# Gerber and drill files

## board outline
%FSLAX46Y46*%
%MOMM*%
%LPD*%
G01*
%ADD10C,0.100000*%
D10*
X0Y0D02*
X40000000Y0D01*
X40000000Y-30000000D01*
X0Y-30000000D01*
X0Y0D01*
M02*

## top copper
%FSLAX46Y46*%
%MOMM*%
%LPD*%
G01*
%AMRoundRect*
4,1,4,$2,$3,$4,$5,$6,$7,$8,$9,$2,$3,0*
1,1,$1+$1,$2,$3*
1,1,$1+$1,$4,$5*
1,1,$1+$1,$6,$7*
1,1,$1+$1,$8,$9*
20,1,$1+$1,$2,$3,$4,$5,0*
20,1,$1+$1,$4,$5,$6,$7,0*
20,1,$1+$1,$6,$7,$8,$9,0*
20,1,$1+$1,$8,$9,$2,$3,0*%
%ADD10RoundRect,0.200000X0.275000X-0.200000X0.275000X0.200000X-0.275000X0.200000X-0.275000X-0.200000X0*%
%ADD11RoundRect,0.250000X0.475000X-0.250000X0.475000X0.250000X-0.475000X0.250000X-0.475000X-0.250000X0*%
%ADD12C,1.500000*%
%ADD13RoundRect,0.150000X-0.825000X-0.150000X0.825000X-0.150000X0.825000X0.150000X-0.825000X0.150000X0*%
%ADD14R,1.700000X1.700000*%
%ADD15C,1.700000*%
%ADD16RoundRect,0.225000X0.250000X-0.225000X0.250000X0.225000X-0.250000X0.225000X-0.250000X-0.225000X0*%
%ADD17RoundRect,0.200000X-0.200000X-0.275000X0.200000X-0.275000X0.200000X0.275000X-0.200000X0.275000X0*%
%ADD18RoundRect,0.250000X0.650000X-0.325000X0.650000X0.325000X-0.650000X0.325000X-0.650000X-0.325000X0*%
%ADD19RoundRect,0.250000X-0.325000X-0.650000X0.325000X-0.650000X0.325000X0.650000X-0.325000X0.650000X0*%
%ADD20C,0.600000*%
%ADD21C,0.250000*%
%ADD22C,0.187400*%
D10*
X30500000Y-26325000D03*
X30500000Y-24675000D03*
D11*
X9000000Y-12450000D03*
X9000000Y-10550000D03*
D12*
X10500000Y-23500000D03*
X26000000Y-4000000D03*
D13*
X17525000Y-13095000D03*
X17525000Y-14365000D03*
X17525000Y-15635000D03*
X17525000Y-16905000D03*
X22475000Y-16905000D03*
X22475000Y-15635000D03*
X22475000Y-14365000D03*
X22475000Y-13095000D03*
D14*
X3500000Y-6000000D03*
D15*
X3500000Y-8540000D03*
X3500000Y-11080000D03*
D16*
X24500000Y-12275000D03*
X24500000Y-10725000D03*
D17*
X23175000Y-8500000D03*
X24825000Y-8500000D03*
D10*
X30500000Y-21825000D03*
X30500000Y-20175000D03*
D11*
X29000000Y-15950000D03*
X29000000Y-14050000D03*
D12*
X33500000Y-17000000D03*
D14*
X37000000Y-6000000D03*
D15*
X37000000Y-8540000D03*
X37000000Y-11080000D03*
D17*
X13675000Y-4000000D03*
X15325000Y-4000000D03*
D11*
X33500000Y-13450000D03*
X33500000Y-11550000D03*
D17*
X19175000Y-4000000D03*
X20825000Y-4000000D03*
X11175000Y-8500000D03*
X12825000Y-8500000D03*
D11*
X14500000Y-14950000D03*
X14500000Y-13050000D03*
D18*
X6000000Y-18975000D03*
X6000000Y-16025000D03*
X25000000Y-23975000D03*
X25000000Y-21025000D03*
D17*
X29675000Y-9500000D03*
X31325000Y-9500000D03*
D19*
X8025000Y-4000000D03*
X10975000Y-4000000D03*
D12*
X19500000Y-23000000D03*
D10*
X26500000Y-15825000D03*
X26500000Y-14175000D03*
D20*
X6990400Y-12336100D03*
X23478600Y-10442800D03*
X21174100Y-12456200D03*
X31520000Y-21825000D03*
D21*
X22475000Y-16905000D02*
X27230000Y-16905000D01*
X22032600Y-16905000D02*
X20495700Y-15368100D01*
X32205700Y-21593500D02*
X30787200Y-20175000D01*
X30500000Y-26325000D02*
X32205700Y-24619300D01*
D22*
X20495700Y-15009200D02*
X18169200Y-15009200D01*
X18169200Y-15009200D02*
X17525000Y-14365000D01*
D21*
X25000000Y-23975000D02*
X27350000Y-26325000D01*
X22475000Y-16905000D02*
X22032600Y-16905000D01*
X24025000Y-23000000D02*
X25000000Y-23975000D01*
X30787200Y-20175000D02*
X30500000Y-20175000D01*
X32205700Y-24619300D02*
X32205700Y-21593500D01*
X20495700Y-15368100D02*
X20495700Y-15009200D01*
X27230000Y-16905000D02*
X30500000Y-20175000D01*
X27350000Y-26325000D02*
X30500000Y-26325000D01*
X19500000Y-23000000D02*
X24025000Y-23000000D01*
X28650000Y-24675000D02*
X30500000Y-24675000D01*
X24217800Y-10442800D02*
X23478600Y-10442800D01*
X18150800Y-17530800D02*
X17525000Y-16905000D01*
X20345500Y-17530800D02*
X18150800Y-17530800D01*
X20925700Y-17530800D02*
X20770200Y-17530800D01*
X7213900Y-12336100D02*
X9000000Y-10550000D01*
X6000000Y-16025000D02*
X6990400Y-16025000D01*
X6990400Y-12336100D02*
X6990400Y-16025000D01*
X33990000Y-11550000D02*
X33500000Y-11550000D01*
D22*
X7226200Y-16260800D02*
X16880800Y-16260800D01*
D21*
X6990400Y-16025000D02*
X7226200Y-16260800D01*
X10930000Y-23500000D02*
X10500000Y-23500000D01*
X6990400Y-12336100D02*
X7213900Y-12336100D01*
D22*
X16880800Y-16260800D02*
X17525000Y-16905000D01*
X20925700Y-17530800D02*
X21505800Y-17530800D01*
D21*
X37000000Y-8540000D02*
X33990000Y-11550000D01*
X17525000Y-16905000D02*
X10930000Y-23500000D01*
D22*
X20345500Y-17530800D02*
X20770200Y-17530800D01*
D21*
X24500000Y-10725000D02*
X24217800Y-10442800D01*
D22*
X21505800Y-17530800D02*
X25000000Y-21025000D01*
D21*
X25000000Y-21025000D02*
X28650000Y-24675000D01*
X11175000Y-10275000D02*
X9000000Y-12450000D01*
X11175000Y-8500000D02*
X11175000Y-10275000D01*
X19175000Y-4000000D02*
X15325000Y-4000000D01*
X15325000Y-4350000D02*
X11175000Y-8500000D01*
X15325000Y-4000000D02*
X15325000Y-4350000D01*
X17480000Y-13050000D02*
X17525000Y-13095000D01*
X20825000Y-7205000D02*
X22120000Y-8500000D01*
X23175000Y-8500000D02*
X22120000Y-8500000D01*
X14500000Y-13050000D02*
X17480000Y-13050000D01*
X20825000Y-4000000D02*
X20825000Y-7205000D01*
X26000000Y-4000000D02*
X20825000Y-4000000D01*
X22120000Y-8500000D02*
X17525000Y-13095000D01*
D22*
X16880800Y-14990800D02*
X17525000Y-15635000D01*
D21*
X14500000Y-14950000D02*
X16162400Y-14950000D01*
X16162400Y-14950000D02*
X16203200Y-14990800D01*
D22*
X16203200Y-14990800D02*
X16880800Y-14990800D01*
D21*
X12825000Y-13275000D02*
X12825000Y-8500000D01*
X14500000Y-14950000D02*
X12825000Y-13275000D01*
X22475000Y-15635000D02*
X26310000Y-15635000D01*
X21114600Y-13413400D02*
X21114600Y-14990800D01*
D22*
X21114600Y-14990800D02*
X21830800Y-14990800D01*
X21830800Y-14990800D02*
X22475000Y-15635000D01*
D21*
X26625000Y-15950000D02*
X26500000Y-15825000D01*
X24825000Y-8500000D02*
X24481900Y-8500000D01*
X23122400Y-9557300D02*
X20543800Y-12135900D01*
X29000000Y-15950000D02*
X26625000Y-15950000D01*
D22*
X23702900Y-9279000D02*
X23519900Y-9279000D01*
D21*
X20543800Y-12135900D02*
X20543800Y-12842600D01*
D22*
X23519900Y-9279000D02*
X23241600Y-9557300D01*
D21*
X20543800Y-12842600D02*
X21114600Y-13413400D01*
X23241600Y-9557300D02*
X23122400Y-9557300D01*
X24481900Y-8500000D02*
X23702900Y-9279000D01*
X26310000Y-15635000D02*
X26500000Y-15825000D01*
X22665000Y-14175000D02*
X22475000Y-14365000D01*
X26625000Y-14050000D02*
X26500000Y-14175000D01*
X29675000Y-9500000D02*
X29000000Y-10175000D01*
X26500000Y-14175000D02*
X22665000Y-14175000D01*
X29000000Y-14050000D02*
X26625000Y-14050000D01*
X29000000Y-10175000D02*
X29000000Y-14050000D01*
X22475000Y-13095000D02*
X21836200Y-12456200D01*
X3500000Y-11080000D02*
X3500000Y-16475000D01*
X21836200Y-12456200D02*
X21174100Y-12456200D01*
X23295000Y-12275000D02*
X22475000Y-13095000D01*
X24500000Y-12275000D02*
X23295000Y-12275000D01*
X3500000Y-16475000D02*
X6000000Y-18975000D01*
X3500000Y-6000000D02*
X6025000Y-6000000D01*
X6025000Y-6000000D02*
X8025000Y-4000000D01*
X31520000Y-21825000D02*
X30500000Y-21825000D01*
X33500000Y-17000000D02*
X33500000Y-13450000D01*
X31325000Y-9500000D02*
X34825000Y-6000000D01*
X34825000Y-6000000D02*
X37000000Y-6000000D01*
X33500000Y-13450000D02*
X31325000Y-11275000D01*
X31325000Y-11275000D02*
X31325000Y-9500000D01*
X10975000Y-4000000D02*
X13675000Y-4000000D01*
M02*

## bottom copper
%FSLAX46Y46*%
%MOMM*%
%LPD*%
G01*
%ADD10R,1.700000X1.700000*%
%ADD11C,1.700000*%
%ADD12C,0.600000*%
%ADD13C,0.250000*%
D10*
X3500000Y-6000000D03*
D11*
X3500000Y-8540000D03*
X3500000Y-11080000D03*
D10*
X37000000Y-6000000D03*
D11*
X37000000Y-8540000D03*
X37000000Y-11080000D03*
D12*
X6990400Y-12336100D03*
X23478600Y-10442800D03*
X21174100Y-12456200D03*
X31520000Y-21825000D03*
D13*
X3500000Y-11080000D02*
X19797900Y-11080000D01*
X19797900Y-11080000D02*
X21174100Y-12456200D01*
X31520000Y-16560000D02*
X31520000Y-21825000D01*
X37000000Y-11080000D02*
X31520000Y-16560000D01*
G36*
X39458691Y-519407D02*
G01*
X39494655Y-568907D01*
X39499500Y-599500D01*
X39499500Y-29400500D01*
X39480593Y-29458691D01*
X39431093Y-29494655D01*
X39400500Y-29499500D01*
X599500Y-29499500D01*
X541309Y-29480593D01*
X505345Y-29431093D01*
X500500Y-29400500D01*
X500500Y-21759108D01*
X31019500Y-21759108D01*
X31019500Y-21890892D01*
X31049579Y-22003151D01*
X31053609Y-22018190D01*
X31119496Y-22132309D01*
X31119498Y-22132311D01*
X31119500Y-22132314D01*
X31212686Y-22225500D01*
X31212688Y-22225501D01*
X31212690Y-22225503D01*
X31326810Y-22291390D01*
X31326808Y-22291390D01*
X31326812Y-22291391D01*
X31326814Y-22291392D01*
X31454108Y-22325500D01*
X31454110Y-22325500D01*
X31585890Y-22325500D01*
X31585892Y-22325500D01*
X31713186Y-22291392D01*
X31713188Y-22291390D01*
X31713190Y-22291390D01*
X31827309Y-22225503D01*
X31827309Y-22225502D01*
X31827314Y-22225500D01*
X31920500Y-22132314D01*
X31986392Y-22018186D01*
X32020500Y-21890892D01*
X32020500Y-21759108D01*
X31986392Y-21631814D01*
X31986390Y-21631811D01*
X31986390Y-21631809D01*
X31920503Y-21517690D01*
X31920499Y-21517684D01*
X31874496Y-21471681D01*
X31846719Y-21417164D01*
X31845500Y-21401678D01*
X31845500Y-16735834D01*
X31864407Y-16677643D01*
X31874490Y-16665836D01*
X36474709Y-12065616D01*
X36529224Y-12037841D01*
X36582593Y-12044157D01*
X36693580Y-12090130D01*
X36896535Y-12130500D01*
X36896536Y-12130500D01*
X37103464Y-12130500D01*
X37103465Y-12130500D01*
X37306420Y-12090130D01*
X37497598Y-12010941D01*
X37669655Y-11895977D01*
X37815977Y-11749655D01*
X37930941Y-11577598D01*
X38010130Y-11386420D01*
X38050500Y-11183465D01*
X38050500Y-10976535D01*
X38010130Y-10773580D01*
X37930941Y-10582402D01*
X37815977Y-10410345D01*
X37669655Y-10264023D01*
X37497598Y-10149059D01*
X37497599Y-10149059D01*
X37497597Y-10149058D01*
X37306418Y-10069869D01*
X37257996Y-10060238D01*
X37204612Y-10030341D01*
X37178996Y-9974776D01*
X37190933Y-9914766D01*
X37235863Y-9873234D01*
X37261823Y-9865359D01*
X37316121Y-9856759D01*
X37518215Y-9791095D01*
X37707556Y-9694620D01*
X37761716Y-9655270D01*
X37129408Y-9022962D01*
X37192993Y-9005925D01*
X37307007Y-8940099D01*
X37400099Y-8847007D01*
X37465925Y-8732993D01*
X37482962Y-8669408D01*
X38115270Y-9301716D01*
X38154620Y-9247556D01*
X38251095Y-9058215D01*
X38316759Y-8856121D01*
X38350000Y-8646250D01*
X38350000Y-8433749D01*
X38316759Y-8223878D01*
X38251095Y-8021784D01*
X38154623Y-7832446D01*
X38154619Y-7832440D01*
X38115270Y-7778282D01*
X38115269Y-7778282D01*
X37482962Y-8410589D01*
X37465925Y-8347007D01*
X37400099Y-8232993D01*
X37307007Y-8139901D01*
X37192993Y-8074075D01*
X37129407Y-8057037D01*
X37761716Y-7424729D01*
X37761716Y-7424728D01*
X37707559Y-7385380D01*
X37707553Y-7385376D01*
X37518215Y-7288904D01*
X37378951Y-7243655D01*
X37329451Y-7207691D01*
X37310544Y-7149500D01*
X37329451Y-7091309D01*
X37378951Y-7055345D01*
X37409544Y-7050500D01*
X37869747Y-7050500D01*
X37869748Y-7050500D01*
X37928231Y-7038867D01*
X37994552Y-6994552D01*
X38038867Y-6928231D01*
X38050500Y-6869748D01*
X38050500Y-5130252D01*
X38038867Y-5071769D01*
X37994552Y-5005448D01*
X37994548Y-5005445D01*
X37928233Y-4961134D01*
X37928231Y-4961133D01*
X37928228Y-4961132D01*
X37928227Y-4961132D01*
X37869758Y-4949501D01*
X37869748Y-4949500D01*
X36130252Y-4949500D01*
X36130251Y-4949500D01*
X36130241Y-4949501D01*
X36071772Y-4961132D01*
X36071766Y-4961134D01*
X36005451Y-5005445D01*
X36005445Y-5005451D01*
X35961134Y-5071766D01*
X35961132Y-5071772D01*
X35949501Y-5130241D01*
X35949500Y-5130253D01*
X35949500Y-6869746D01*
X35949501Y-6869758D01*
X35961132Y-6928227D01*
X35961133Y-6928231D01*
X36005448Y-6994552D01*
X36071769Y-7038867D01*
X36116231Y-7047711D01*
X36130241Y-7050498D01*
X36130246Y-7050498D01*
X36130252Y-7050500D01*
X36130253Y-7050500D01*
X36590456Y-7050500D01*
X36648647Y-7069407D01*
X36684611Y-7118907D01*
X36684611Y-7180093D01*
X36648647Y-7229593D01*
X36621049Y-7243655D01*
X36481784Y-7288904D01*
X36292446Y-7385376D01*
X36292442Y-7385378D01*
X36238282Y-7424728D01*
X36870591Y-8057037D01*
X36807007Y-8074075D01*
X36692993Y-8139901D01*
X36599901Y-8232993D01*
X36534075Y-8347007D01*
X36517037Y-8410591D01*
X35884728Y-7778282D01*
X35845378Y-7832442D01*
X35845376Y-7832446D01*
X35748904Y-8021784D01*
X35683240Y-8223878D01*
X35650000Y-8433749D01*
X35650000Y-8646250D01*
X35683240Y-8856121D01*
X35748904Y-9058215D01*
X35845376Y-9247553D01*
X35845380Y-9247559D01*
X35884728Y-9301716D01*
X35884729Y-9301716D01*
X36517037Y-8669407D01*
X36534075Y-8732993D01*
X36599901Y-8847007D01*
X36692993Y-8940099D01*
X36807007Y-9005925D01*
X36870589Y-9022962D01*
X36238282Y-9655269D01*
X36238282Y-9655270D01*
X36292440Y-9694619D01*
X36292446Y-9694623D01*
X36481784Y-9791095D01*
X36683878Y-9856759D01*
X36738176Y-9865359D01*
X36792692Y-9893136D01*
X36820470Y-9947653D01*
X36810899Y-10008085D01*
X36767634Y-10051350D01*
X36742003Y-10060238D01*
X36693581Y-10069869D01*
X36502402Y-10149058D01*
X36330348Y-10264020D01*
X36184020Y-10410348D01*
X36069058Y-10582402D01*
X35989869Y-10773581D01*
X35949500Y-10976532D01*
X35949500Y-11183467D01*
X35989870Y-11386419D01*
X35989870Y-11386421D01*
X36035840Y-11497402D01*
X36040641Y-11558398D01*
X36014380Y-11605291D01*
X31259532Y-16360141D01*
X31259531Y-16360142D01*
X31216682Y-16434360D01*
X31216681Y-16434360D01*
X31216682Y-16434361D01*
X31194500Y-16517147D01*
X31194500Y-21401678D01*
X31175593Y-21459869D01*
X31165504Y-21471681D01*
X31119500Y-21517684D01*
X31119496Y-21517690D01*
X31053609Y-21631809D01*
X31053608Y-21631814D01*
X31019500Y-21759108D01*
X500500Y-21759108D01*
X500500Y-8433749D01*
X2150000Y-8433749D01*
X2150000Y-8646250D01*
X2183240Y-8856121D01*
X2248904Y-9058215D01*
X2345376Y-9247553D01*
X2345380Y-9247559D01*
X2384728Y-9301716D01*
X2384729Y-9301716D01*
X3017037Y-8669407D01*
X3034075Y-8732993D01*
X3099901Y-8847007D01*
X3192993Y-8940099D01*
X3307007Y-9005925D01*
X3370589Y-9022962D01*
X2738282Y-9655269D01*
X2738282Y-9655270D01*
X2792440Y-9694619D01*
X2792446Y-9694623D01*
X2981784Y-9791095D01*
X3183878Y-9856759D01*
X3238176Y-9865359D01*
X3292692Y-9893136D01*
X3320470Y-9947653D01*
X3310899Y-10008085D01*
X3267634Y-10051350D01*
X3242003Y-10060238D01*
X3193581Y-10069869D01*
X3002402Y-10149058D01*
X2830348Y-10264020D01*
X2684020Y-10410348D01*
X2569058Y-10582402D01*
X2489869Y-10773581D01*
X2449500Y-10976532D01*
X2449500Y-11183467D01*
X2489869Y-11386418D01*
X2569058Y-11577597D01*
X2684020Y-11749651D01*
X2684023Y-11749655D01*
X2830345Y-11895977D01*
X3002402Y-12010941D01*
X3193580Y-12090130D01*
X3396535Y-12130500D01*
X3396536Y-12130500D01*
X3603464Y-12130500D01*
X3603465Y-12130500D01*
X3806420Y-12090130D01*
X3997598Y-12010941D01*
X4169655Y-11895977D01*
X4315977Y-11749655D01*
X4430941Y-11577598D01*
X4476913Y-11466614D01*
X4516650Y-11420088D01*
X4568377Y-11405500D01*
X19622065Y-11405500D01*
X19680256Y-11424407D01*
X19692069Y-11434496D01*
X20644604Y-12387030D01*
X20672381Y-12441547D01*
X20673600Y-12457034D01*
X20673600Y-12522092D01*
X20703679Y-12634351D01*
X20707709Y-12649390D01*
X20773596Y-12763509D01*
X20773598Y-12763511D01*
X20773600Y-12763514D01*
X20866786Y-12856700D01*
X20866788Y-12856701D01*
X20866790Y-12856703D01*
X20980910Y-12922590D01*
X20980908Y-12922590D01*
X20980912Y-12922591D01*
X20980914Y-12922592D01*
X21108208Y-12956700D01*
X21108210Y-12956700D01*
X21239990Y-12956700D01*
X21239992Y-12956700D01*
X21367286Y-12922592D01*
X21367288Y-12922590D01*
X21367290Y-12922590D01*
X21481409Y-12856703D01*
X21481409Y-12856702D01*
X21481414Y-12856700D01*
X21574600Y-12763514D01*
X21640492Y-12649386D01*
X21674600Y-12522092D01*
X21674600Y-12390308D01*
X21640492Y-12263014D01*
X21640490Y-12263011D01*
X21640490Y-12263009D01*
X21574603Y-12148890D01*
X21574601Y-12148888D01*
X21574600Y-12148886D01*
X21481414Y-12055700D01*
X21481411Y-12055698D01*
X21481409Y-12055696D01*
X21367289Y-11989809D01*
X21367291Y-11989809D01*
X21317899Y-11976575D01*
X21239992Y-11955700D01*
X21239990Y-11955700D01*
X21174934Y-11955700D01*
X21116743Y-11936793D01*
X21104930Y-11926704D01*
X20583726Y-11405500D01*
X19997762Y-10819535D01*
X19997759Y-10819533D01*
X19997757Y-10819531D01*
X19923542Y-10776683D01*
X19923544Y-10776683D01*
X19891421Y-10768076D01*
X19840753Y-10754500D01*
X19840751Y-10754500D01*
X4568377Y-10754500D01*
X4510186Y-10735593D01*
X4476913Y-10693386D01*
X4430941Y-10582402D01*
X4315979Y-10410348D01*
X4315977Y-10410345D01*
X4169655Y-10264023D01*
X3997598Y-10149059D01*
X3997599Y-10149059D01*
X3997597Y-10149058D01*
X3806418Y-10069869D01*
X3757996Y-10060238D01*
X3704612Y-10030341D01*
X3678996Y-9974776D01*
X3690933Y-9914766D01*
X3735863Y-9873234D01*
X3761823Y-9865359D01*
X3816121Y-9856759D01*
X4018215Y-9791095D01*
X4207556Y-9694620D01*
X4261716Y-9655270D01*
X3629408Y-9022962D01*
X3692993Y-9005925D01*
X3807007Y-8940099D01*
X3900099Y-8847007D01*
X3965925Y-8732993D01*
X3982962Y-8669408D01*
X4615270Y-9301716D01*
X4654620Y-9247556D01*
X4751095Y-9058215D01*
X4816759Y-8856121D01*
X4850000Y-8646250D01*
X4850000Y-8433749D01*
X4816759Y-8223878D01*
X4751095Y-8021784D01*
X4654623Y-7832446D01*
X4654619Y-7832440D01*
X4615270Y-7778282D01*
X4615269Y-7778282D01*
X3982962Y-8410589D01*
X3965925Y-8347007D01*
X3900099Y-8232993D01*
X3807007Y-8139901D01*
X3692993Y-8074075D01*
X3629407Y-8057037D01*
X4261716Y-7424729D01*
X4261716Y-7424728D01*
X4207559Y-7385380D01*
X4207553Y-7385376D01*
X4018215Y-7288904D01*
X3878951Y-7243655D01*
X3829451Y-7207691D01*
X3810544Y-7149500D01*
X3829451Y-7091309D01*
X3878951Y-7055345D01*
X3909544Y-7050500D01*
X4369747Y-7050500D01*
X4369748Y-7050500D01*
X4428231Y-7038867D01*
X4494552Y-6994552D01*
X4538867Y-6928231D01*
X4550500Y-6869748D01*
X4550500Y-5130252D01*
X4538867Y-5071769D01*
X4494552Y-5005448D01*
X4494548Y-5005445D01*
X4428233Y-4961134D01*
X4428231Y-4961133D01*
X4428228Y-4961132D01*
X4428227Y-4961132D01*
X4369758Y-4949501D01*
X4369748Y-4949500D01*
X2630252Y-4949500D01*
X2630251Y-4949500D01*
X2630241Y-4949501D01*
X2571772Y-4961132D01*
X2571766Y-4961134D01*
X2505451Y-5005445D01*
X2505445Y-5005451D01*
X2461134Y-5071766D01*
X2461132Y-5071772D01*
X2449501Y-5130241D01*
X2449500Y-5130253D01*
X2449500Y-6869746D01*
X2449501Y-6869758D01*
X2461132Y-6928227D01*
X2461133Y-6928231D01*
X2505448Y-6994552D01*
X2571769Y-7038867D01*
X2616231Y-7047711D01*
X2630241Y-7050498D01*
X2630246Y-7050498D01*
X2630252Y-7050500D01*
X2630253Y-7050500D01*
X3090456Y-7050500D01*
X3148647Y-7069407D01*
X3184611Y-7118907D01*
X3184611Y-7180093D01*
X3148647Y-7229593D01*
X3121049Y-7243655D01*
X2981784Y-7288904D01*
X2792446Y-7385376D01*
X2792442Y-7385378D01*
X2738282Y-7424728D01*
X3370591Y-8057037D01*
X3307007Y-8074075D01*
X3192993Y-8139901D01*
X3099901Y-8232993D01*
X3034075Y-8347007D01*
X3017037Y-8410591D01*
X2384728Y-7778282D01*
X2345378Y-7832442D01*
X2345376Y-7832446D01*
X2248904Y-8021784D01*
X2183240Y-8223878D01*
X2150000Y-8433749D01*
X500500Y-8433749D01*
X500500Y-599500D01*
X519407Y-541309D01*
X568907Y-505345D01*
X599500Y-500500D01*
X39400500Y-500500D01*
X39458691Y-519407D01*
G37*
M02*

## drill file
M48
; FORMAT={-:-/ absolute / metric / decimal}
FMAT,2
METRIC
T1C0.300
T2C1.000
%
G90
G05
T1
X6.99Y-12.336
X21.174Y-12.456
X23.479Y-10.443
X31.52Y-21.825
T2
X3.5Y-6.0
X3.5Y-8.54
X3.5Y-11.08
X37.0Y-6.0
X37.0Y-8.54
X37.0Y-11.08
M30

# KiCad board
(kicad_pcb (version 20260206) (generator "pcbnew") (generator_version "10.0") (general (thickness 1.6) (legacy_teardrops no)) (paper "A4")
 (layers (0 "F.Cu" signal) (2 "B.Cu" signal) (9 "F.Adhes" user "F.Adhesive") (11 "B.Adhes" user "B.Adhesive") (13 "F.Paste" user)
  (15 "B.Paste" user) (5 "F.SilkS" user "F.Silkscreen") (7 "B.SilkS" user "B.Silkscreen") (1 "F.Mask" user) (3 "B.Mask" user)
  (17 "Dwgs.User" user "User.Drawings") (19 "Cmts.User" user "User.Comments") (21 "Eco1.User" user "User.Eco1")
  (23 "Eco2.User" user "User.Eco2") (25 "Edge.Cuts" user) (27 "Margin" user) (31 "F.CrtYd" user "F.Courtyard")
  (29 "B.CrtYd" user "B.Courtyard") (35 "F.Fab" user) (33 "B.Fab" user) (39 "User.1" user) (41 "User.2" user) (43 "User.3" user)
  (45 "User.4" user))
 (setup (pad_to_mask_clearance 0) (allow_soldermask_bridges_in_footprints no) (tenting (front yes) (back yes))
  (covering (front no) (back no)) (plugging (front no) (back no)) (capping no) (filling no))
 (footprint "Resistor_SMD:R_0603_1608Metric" (layer "F.Cu") (at 30.5 25.5 90)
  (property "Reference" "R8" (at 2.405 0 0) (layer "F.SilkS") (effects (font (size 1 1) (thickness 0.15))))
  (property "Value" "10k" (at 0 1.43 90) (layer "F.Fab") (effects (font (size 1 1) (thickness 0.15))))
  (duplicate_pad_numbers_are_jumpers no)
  (pad "1" smd roundrect (at -0.825 0 90) (size 0.8 0.95) (layers "F.Cu" "F.Mask" "F.Paste") (roundrect_rratio 0.25) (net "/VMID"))
  (pad "2" smd roundrect (at 0.825 0 90) (size 0.8 0.95) (layers "F.Cu" "F.Mask" "F.Paste") (roundrect_rratio 0.25) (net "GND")))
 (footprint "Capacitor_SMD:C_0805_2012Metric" (layer "F.Cu") (at 9 11.5 90)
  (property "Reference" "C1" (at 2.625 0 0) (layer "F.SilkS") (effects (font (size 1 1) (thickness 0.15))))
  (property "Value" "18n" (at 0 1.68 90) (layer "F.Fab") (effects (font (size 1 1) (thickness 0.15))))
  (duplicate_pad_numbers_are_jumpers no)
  (pad "1" smd roundrect (at -0.95 0 90) (size 1 1.45) (layers "F.Cu" "F.Mask" "F.Paste") (roundrect_rratio 0.25) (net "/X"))
  (pad "2" smd roundrect (at 0.95 0 90) (size 1 1.45) (layers "F.Cu" "F.Mask" "F.Paste") (roundrect_rratio 0.25) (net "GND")))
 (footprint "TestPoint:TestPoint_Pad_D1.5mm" (layer "F.Cu") (at 10.5 23.5)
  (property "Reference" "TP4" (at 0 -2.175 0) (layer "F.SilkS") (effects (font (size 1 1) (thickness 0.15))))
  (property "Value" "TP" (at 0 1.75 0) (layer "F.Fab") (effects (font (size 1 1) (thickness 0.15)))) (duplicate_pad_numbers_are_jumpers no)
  (pad "1" smd circle (at 0 0) (size 1.5 1.5) (layers "F.Cu" "F.Mask") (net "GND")))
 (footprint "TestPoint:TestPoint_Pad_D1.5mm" (layer "F.Cu") (at 26 4)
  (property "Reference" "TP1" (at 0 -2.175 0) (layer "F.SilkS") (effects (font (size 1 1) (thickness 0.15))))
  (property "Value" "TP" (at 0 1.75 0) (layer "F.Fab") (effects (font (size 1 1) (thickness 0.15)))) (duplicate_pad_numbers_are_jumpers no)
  (pad "1" smd circle (at 0 0) (size 1.5 1.5) (layers "F.Cu" "F.Mask") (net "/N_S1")))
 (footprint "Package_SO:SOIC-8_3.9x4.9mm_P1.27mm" (layer "F.Cu") (at 20 15)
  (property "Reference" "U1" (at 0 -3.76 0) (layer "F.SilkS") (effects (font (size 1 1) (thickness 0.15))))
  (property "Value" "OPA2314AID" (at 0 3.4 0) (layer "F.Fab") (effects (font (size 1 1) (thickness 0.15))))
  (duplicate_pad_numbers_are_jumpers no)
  (pad "1" smd roundrect (at -2.475 -1.905) (size 1.95 0.6) (layers "F.Cu" "F.Mask" "F.Paste") (roundrect_rratio 0.25) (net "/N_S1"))
  (pad "2" smd roundrect (at -2.475 -0.635) (size 1.95 0.6) (layers "F.Cu" "F.Mask" "F.Paste") (roundrect_rratio 0.25) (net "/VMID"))
  (pad "3" smd roundrect (at -2.475 0.635) (size 1.95 0.6) (layers "F.Cu" "F.Mask" "F.Paste") (roundrect_rratio 0.25) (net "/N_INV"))
  (pad "4" smd roundrect (at -2.475 1.905) (size 1.95 0.6) (layers "F.Cu" "F.Mask" "F.Paste") (roundrect_rratio 0.25) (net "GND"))
  (pad "5" smd roundrect (at 2.475 1.905) (size 1.95 0.6) (layers "F.Cu" "F.Mask" "F.Paste") (roundrect_rratio 0.25) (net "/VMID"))
  (pad "6" smd roundrect (at 2.475 0.635) (size 1.95 0.6) (layers "F.Cu" "F.Mask" "F.Paste") (roundrect_rratio 0.25) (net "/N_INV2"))
  (pad "7" smd roundrect (at 2.475 -0.635) (size 1.95 0.6) (layers "F.Cu" "F.Mask" "F.Paste") (roundrect_rratio 0.25) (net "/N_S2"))
  (pad "8" smd roundrect (at 2.475 -1.905) (size 1.95 0.6) (layers "F.Cu" "F.Mask" "F.Paste") (roundrect_rratio 0.25) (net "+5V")))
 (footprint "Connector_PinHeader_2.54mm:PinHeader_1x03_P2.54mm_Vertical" (layer "F.Cu") (at 3.5 6)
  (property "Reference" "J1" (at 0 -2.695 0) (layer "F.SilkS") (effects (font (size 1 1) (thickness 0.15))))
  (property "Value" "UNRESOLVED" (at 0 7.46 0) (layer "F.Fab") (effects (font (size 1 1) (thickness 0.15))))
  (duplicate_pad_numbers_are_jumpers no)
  (pad "1" thru_hole rect (at 0 0) (size 1.7 1.7) (drill 1) (layers "*.Cu" "*.Mask") (remove_unused_layers no) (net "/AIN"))
  (pad "2" thru_hole circle (at 0 2.54) (size 1.7 1.7) (drill 1) (layers "*.Cu" "*.Mask") (remove_unused_layers no) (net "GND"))
  (pad "3" thru_hole circle (at 0 5.08) (size 1.7 1.7) (drill 1) (layers "*.Cu" "*.Mask") (remove_unused_layers no) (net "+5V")))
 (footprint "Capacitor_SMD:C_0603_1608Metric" (layer "F.Cu") (at 24.5 11.5 90)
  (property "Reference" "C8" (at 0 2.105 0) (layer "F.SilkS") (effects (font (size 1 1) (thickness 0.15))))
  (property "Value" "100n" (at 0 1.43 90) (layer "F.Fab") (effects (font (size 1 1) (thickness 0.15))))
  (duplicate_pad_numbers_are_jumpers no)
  (pad "1" smd roundrect (at -0.775 0 90) (size 0.9 0.95) (layers "F.Cu" "F.Mask" "F.Paste") (roundrect_rratio 0.25) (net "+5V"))
  (pad "2" smd roundrect (at 0.775 0 90) (size 0.9 0.95) (layers "F.Cu" "F.Mask" "F.Paste") (roundrect_rratio 0.25) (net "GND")))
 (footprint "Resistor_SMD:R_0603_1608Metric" (layer "F.Cu") (at 24 8.5)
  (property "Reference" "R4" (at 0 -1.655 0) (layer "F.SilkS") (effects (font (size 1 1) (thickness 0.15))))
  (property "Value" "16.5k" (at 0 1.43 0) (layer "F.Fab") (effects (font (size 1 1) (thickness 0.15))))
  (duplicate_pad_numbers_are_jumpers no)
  (pad "1" smd roundrect (at -0.825 0) (size 0.8 0.95) (layers "F.Cu" "F.Mask" "F.Paste") (roundrect_rratio 0.25) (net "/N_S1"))
  (pad "2" smd roundrect (at 0.825 0) (size 0.8 0.95) (layers "F.Cu" "F.Mask" "F.Paste") (roundrect_rratio 0.25) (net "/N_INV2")))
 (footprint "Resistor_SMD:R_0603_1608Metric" (layer "F.Cu") (at 30.5 21 90)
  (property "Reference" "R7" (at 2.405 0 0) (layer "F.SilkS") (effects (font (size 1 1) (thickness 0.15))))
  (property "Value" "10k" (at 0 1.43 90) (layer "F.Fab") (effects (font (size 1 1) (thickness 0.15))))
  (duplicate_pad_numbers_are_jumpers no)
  (pad "1" smd roundrect (at -0.825 0 90) (size 0.8 0.95) (layers "F.Cu" "F.Mask" "F.Paste") (roundrect_rratio 0.25) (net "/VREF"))
  (pad "2" smd roundrect (at 0.825 0 90) (size 0.8 0.95) (layers "F.Cu" "F.Mask" "F.Paste") (roundrect_rratio 0.25) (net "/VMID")))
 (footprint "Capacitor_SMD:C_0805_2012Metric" (layer "F.Cu") (at 29 15 90)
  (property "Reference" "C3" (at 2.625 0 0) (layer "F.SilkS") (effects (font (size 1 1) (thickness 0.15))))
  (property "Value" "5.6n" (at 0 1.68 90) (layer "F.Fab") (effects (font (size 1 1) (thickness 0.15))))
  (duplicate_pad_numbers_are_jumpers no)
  (pad "1" smd roundrect (at -0.95 0 90) (size 1 1.45) (layers "F.Cu" "F.Mask" "F.Paste") (roundrect_rratio 0.25) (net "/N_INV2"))
  (pad "2" smd roundrect (at 0.95 0 90) (size 1 1.45) (layers "F.Cu" "F.Mask" "F.Paste") (roundrect_rratio 0.25) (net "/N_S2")))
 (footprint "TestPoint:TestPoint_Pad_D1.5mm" (layer "F.Cu") (at 33.5 17)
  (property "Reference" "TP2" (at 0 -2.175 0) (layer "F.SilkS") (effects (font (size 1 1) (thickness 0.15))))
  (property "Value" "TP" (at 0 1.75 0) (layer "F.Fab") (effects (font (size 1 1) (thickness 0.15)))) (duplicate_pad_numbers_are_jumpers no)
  (pad "1" smd circle (at 0 0) (size 1.5 1.5) (layers "F.Cu" "F.Mask") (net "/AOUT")))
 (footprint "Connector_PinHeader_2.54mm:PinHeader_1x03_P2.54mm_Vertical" (layer "F.Cu") (at 37 6)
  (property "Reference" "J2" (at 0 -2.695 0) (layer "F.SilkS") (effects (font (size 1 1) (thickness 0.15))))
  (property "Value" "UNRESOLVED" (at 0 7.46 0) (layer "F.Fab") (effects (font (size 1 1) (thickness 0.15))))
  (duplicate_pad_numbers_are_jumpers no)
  (pad "1" thru_hole rect (at 0 0) (size 1.7 1.7) (drill 1) (layers "*.Cu" "*.Mask") (remove_unused_layers no) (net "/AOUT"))
  (pad "2" thru_hole circle (at 0 2.54) (size 1.7 1.7) (drill 1) (layers "*.Cu" "*.Mask") (remove_unused_layers no) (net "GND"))
  (pad "3" thru_hole circle (at 0 5.08) (size 1.7 1.7) (drill 1) (layers "*.Cu" "*.Mask") (remove_unused_layers no) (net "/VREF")))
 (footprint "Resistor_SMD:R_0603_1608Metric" (layer "F.Cu") (at 14.5 4)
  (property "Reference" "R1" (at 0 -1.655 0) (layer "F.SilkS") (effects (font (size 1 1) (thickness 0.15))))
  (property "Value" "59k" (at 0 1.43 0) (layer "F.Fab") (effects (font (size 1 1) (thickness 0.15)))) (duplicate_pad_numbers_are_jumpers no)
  (pad "1" smd roundrect (at -0.825 0) (size 0.8 0.95) (layers "F.Cu" "F.Mask" "F.Paste") (roundrect_rratio 0.25) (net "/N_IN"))
  (pad "2" smd roundrect (at 0.825 0) (size 0.8 0.95) (layers "F.Cu" "F.Mask" "F.Paste") (roundrect_rratio 0.25) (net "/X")))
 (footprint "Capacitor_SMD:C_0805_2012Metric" (layer "F.Cu") (at 33.5 12.5 90)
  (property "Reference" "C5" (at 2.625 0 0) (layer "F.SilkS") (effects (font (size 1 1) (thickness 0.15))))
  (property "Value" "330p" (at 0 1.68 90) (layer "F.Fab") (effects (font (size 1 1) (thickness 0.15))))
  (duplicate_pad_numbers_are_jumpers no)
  (pad "1" smd roundrect (at -0.95 0 90) (size 1 1.45) (layers "F.Cu" "F.Mask" "F.Paste") (roundrect_rratio 0.25) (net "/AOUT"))
  (pad "2" smd roundrect (at 0.95 0 90) (size 1 1.45) (layers "F.Cu" "F.Mask" "F.Paste") (roundrect_rratio 0.25) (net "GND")))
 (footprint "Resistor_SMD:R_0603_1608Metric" (layer "F.Cu") (at 20 4)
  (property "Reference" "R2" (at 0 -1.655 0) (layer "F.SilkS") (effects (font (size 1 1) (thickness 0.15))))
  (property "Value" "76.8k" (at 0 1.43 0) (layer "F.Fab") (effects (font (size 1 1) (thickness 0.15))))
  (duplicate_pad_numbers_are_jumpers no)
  (pad "1" smd roundrect (at -0.825 0) (size 0.8 0.95) (layers "F.Cu" "F.Mask" "F.Paste") (roundrect_rratio 0.25) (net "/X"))
  (pad "2" smd roundrect (at 0.825 0) (size 0.8 0.95) (layers "F.Cu" "F.Mask" "F.Paste") (roundrect_rratio 0.25) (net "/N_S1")))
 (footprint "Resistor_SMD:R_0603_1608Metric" (layer "F.Cu") (at 12 8.5)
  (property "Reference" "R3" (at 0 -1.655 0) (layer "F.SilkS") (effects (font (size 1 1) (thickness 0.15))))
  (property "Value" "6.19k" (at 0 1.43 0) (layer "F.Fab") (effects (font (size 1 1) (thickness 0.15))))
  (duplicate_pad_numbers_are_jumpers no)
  (pad "1" smd roundrect (at -0.825 0) (size 0.8 0.95) (layers "F.Cu" "F.Mask" "F.Paste") (roundrect_rratio 0.25) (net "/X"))
  (pad "2" smd roundrect (at 0.825 0) (size 0.8 0.95) (layers "F.Cu" "F.Mask" "F.Paste") (roundrect_rratio 0.25) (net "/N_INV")))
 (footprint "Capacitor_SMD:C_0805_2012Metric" (layer "F.Cu") (at 14.5 14 90)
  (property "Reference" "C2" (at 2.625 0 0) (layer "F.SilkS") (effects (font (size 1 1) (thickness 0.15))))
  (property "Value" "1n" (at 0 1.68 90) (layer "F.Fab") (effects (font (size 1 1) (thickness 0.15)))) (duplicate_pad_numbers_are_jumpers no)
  (pad "1" smd roundrect (at -0.95 0 90) (size 1 1.45) (layers "F.Cu" "F.Mask" "F.Paste") (roundrect_rratio 0.25) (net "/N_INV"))
  (pad "2" smd roundrect (at 0.95 0 90) (size 1 1.45) (layers "F.Cu" "F.Mask" "F.Paste") (roundrect_rratio 0.25) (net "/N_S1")))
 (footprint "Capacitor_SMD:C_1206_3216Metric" (layer "F.Cu") (at 6 17.5 90)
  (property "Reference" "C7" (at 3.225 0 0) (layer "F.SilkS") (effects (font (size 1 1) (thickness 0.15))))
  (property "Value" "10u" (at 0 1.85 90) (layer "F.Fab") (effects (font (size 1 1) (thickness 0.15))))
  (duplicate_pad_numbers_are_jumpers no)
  (pad "1" smd roundrect (at -1.475 0 90) (size 1.15 1.8) (layers "F.Cu" "F.Mask" "F.Paste") (roundrect_rratio 0.217391) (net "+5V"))
  (pad "2" smd roundrect (at 1.475 0 90) (size 1.15 1.8) (layers "F.Cu" "F.Mask" "F.Paste") (roundrect_rratio 0.217391) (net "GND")))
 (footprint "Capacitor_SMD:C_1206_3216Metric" (layer "F.Cu") (at 25 22.5 90)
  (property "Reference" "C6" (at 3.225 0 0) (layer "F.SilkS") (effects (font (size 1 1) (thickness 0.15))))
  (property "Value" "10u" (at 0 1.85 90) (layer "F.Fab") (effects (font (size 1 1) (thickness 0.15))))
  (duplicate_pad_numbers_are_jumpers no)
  (pad "1" smd roundrect (at -1.475 0 90) (size 1.15 1.8) (layers "F.Cu" "F.Mask" "F.Paste") (roundrect_rratio 0.217391) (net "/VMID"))
  (pad "2" smd roundrect (at 1.475 0 90) (size 1.15 1.8) (layers "F.Cu" "F.Mask" "F.Paste") (roundrect_rratio 0.217391) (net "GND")))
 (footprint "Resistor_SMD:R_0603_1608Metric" (layer "F.Cu") (at 30.5 9.5)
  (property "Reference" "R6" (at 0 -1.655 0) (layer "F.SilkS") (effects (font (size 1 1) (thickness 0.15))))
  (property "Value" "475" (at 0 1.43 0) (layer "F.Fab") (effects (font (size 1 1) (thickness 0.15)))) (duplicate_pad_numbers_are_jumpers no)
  (pad "1" smd roundrect (at -0.825 0) (size 0.8 0.95) (layers "F.Cu" "F.Mask" "F.Paste") (roundrect_rratio 0.25) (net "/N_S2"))
  (pad "2" smd roundrect (at 0.825 0) (size 0.8 0.95) (layers "F.Cu" "F.Mask" "F.Paste") (roundrect_rratio 0.25) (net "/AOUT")))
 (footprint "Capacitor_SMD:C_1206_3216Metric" (layer "F.Cu") (at 9.5 4)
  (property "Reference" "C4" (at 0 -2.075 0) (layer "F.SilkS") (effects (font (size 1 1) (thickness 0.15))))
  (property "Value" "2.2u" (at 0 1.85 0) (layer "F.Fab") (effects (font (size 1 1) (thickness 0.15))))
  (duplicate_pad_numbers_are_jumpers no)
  (pad "1" smd roundrect (at -1.475 0) (size 1.15 1.8) (layers "F.Cu" "F.Mask" "F.Paste") (roundrect_rratio 0.217391) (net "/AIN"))
  (pad "2" smd roundrect (at 1.475 0) (size 1.15 1.8) (layers "F.Cu" "F.Mask" "F.Paste") (roundrect_rratio 0.217391) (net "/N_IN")))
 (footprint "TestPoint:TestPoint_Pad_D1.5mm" (layer "F.Cu") (at 19.5 23)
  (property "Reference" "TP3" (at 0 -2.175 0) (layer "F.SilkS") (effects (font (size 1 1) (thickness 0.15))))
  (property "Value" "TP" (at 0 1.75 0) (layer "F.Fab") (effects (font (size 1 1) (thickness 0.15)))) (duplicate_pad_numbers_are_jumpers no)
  (pad "1" smd circle (at 0 0) (size 1.5 1.5) (layers "F.Cu" "F.Mask") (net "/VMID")))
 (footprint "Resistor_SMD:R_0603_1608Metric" (layer "F.Cu") (at 26.5 15 90)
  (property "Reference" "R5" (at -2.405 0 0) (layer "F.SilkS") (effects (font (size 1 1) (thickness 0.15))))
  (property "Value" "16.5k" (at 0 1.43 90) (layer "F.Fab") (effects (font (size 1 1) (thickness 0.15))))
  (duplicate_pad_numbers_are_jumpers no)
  (pad "1" smd roundrect (at -0.825 0 90) (size 0.8 0.95) (layers "F.Cu" "F.Mask" "F.Paste") (roundrect_rratio 0.25) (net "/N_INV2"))
  (pad "2" smd roundrect (at 0.825 0 90) (size 0.8 0.95) (layers "F.Cu" "F.Mask" "F.Paste") (roundrect_rratio 0.25) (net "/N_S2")))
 (gr_rect (start 0 0) (end 40 30) (stroke (width 0.1) (type default)) (fill no) (layer "Edge.Cuts"))
 (segment (start 22.475 16.905) (end 27.23 16.905) (width 0.25) (layer "F.Cu") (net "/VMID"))
 (segment (start 22.0326 16.905) (end 20.4957 15.3681) (width 0.25) (layer "F.Cu") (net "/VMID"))
 (segment (start 32.2057 21.5935) (end 30.7872 20.175) (width 0.25) (layer "F.Cu") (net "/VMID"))
 (segment (start 30.5 26.325) (end 32.2057 24.6193) (width 0.25) (layer "F.Cu") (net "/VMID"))
 (segment (start 20.4957 15.0092) (end 18.1692 15.0092) (width 0.1874) (layer "F.Cu") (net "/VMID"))
 (segment (start 18.1692 15.0092) (end 17.525 14.365) (width 0.1874) (layer "F.Cu") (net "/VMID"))
 (segment (start 25 23.975) (end 27.35 26.325) (width 0.25) (layer "F.Cu") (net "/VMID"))
 (segment (start 22.475 16.905) (end 22.0326 16.905) (width 0.25) (layer "F.Cu") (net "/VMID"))
 (segment (start 24.025 23) (end 25 23.975) (width 0.25) (layer "F.Cu") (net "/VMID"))
 (segment (start 30.7872 20.175) (end 30.5 20.175) (width 0.25) (layer "F.Cu") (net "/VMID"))
 (segment (start 32.2057 24.6193) (end 32.2057 21.5935) (width 0.25) (layer "F.Cu") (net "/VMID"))
 (segment (start 20.4957 15.3681) (end 20.4957 15.0092) (width 0.25) (layer "F.Cu") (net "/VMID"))
 (segment (start 27.23 16.905) (end 30.5 20.175) (width 0.25) (layer "F.Cu") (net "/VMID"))
 (segment (start 27.35 26.325) (end 30.5 26.325) (width 0.25) (layer "F.Cu") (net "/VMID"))
 (segment (start 19.5 23) (end 24.025 23) (width 0.25) (layer "F.Cu") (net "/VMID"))
 (segment (start 28.65 24.675) (end 30.5 24.675) (width 0.25) (layer "F.Cu") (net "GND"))
 (segment (start 24.2178 10.4428) (end 23.4786 10.4428) (width 0.25) (layer "F.Cu") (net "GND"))
 (segment (start 18.1508 17.5308) (end 17.525 16.905) (width 0.25) (layer "F.Cu") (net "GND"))
 (segment (start 20.3455 17.5308) (end 18.1508 17.5308) (width 0.25) (layer "F.Cu") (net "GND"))
 (segment (start 20.9257 17.5308) (end 20.7702 17.5308) (width 0.25) (layer "F.Cu") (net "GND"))
 (segment (start 7.2139 12.3361) (end 9 10.55) (width 0.25) (layer "F.Cu") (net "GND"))
 (segment (start 6 16.025) (end 6.9904 16.025) (width 0.25) (layer "F.Cu") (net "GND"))
 (segment (start 6.9904 12.3361) (end 6.9904 16.025) (width 0.25) (layer "F.Cu") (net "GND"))
 (segment (start 33.99 11.55) (end 33.5 11.55) (width 0.25) (layer "F.Cu") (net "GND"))
 (segment (start 7.2262 16.2608) (end 16.8808 16.2608) (width 0.1874) (layer "F.Cu") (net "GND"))
 (segment (start 6.9904 16.025) (end 7.2262 16.2608) (width 0.25) (layer "F.Cu") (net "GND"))
 (segment (start 10.93 23.5) (end 10.5 23.5) (width 0.25) (layer "F.Cu") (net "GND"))
 (segment (start 6.9904 12.3361) (end 7.2139 12.3361) (width 0.25) (layer "F.Cu") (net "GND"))
 (segment (start 16.8808 16.2608) (end 17.525 16.905) (width 0.1874) (layer "F.Cu") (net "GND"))
 (segment (start 20.9257 17.5308) (end 21.5058 17.5308) (width 0.1874) (layer "F.Cu") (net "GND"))
 (segment (start 37 8.54) (end 33.99 11.55) (width 0.25) (layer "F.Cu") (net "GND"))
 (segment (start 17.525 16.905) (end 10.93 23.5) (width 0.25) (layer "F.Cu") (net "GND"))
 (segment (start 20.3455 17.5308) (end 20.7702 17.5308) (width 0.1874) (layer "F.Cu") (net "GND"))
 (segment (start 24.5 10.725) (end 24.2178 10.4428) (width 0.25) (layer "F.Cu") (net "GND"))
 (segment (start 21.5058 17.5308) (end 25 21.025) (width 0.1874) (layer "F.Cu") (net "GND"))
 (segment (start 25 21.025) (end 28.65 24.675) (width 0.25) (layer "F.Cu") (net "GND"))
 (via (at 6.9904 12.3361) (size 0.6) (drill 0.3) (layers "F.Cu" "B.Cu") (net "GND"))
 (via (at 23.4786 10.4428) (size 0.6) (drill 0.3) (layers "F.Cu" "B.Cu") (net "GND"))
 (segment (start 11.175 10.275) (end 9 12.45) (width 0.25) (layer "F.Cu") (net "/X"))
 (segment (start 11.175 8.5) (end 11.175 10.275) (width 0.25) (layer "F.Cu") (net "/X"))
 (segment (start 19.175 4) (end 15.325 4) (width 0.25) (layer "F.Cu") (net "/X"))
 (segment (start 15.325 4.35) (end 11.175 8.5) (width 0.25) (layer "F.Cu") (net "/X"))
 (segment (start 15.325 4) (end 15.325 4.35) (width 0.25) (layer "F.Cu") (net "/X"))
 (segment (start 17.48 13.05) (end 17.525 13.095) (width 0.25) (layer "F.Cu") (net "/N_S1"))
 (segment (start 20.825 7.205) (end 22.12 8.5) (width 0.25) (layer "F.Cu") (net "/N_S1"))
 (segment (start 23.175 8.5) (end 22.12 8.5) (width 0.25) (layer "F.Cu") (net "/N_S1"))
 (segment (start 14.5 13.05) (end 17.48 13.05) (width 0.25) (layer "F.Cu") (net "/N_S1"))
 (segment (start 20.825 4) (end 20.825 7.205) (width 0.25) (layer "F.Cu") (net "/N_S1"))
 (segment (start 26 4) (end 20.825 4) (width 0.25) (layer "F.Cu") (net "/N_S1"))
 (segment (start 22.12 8.5) (end 17.525 13.095) (width 0.25) (layer "F.Cu") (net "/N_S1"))
 (segment (start 16.8808 14.9908) (end 17.525 15.635) (width 0.1874) (layer "F.Cu") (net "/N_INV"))
 (segment (start 14.5 14.95) (end 16.1624 14.95) (width 0.25) (layer "F.Cu") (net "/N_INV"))
 (segment (start 16.1624 14.95) (end 16.2032 14.9908) (width 0.25) (layer "F.Cu") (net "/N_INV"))
 (segment (start 16.2032 14.9908) (end 16.8808 14.9908) (width 0.1874) (layer "F.Cu") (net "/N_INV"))
 (segment (start 12.825 13.275) (end 12.825 8.5) (width 0.25) (layer "F.Cu") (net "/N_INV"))
 (segment (start 14.5 14.95) (end 12.825 13.275) (width 0.25) (layer "F.Cu") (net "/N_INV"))
 (segment (start 22.475 15.635) (end 26.31 15.635) (width 0.25) (layer "F.Cu") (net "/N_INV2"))
 (segment (start 21.1146 13.4134) (end 21.1146 14.9908) (width 0.25) (layer "F.Cu") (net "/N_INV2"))
 (segment (start 21.1146 14.9908) (end 21.8308 14.9908) (width 0.1874) (layer "F.Cu") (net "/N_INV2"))
 (segment (start 21.8308 14.9908) (end 22.475 15.635) (width 0.1874) (layer "F.Cu") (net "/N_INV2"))
 (segment (start 26.625 15.95) (end 26.5 15.825) (width 0.25) (layer "F.Cu") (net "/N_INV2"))
 (segment (start 24.825 8.5) (end 24.4819 8.5) (width 0.25) (layer "F.Cu") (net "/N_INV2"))
 (segment (start 23.1224 9.5573) (end 20.5438 12.1359) (width 0.25) (layer "F.Cu") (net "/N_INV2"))
 (segment (start 29 15.95) (end 26.625 15.95) (width 0.25) (layer "F.Cu") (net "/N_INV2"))
 (segment (start 23.7029 9.279) (end 23.5199 9.279) (width 0.1874) (layer "F.Cu") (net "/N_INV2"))
 (segment (start 20.5438 12.1359) (end 20.5438 12.8426) (width 0.25) (layer "F.Cu") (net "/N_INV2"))
 (segment (start 23.5199 9.279) (end 23.2416 9.5573) (width 0.1874) (layer "F.Cu") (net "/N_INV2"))
 (segment (start 20.5438 12.8426) (end 21.1146 13.4134) (width 0.25) (layer "F.Cu") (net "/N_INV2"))
 (segment (start 23.2416 9.5573) (end 23.1224 9.5573) (width 0.25) (layer "F.Cu") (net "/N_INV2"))
 (segment (start 24.4819 8.5) (end 23.7029 9.279) (width 0.25) (layer "F.Cu") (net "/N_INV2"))
 (segment (start 26.31 15.635) (end 26.5 15.825) (width 0.25) (layer "F.Cu") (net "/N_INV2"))
 (segment (start 22.665 14.175) (end 22.475 14.365) (width 0.25) (layer "F.Cu") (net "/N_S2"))
 (segment (start 26.625 14.05) (end 26.5 14.175) (width 0.25) (layer "F.Cu") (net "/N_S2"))
 (segment (start 29.675 9.5) (end 29 10.175) (width 0.25) (layer "F.Cu") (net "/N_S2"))
 (segment (start 26.5 14.175) (end 22.665 14.175) (width 0.25) (layer "F.Cu") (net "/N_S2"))
 (segment (start 29 14.05) (end 26.625 14.05) (width 0.25) (layer "F.Cu") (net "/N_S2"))
 (segment (start 29 10.175) (end 29 14.05) (width 0.25) (layer "F.Cu") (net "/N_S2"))
 (segment (start 22.475 13.095) (end 21.8362 12.4562) (width 0.25) (layer "F.Cu") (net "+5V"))
 (segment (start 3.5 11.08) (end 3.5 16.475) (width 0.25) (layer "F.Cu") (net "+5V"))
 (segment (start 21.8362 12.4562) (end 21.1741 12.4562) (width 0.25) (layer "F.Cu") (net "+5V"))
 (segment (start 23.295 12.275) (end 22.475 13.095) (width 0.25) (layer "F.Cu") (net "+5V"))
 (segment (start 24.5 12.275) (end 23.295 12.275) (width 0.25) (layer "F.Cu") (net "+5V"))
 (segment (start 3.5 16.475) (end 6 18.975) (width 0.25) (layer "F.Cu") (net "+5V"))
 (via (at 21.1741 12.4562) (size 0.6) (drill 0.3) (layers "F.Cu" "B.Cu") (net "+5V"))
 (segment (start 3.5 11.08) (end 19.7979 11.08) (width 0.25) (layer "B.Cu") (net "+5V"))
 (segment (start 19.7979 11.08) (end 21.1741 12.4562) (width 0.25) (layer "B.Cu") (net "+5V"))
 (segment (start 3.5 6) (end 6.025 6) (width 0.25) (layer "F.Cu") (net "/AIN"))
 (segment (start 6.025 6) (end 8.025 4) (width 0.25) (layer "F.Cu") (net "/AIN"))
 (segment (start 31.52 21.825) (end 30.5 21.825) (width 0.25) (layer "F.Cu") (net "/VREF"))
 (via (at 31.52 21.825) (size 0.6) (drill 0.3) (layers "F.Cu" "B.Cu") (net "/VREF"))
 (segment (start 31.52 16.56) (end 31.52 21.825) (width 0.25) (layer "B.Cu") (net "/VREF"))
 (segment (start 37 11.08) (end 31.52 16.56) (width 0.25) (layer "B.Cu") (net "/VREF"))
 (segment (start 33.5 17) (end 33.5 13.45) (width 0.25) (layer "F.Cu") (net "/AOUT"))
 (segment (start 31.325 9.5) (end 34.825 6) (width 0.25) (layer "F.Cu") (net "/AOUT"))
 (segment (start 34.825 6) (end 37 6) (width 0.25) (layer "F.Cu") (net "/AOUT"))
 (segment (start 33.5 13.45) (end 31.325 11.275) (width 0.25) (layer "F.Cu") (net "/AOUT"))
 (segment (start 31.325 11.275) (end 31.325 9.5) (width 0.25) (layer "F.Cu") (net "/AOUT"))
 (segment (start 10.975 4) (end 13.675 4) (width 0.25) (layer "F.Cu") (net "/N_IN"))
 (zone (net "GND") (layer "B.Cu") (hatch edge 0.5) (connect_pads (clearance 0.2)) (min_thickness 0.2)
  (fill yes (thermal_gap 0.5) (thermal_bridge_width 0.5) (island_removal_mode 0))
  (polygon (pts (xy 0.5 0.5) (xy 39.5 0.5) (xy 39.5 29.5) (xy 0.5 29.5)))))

